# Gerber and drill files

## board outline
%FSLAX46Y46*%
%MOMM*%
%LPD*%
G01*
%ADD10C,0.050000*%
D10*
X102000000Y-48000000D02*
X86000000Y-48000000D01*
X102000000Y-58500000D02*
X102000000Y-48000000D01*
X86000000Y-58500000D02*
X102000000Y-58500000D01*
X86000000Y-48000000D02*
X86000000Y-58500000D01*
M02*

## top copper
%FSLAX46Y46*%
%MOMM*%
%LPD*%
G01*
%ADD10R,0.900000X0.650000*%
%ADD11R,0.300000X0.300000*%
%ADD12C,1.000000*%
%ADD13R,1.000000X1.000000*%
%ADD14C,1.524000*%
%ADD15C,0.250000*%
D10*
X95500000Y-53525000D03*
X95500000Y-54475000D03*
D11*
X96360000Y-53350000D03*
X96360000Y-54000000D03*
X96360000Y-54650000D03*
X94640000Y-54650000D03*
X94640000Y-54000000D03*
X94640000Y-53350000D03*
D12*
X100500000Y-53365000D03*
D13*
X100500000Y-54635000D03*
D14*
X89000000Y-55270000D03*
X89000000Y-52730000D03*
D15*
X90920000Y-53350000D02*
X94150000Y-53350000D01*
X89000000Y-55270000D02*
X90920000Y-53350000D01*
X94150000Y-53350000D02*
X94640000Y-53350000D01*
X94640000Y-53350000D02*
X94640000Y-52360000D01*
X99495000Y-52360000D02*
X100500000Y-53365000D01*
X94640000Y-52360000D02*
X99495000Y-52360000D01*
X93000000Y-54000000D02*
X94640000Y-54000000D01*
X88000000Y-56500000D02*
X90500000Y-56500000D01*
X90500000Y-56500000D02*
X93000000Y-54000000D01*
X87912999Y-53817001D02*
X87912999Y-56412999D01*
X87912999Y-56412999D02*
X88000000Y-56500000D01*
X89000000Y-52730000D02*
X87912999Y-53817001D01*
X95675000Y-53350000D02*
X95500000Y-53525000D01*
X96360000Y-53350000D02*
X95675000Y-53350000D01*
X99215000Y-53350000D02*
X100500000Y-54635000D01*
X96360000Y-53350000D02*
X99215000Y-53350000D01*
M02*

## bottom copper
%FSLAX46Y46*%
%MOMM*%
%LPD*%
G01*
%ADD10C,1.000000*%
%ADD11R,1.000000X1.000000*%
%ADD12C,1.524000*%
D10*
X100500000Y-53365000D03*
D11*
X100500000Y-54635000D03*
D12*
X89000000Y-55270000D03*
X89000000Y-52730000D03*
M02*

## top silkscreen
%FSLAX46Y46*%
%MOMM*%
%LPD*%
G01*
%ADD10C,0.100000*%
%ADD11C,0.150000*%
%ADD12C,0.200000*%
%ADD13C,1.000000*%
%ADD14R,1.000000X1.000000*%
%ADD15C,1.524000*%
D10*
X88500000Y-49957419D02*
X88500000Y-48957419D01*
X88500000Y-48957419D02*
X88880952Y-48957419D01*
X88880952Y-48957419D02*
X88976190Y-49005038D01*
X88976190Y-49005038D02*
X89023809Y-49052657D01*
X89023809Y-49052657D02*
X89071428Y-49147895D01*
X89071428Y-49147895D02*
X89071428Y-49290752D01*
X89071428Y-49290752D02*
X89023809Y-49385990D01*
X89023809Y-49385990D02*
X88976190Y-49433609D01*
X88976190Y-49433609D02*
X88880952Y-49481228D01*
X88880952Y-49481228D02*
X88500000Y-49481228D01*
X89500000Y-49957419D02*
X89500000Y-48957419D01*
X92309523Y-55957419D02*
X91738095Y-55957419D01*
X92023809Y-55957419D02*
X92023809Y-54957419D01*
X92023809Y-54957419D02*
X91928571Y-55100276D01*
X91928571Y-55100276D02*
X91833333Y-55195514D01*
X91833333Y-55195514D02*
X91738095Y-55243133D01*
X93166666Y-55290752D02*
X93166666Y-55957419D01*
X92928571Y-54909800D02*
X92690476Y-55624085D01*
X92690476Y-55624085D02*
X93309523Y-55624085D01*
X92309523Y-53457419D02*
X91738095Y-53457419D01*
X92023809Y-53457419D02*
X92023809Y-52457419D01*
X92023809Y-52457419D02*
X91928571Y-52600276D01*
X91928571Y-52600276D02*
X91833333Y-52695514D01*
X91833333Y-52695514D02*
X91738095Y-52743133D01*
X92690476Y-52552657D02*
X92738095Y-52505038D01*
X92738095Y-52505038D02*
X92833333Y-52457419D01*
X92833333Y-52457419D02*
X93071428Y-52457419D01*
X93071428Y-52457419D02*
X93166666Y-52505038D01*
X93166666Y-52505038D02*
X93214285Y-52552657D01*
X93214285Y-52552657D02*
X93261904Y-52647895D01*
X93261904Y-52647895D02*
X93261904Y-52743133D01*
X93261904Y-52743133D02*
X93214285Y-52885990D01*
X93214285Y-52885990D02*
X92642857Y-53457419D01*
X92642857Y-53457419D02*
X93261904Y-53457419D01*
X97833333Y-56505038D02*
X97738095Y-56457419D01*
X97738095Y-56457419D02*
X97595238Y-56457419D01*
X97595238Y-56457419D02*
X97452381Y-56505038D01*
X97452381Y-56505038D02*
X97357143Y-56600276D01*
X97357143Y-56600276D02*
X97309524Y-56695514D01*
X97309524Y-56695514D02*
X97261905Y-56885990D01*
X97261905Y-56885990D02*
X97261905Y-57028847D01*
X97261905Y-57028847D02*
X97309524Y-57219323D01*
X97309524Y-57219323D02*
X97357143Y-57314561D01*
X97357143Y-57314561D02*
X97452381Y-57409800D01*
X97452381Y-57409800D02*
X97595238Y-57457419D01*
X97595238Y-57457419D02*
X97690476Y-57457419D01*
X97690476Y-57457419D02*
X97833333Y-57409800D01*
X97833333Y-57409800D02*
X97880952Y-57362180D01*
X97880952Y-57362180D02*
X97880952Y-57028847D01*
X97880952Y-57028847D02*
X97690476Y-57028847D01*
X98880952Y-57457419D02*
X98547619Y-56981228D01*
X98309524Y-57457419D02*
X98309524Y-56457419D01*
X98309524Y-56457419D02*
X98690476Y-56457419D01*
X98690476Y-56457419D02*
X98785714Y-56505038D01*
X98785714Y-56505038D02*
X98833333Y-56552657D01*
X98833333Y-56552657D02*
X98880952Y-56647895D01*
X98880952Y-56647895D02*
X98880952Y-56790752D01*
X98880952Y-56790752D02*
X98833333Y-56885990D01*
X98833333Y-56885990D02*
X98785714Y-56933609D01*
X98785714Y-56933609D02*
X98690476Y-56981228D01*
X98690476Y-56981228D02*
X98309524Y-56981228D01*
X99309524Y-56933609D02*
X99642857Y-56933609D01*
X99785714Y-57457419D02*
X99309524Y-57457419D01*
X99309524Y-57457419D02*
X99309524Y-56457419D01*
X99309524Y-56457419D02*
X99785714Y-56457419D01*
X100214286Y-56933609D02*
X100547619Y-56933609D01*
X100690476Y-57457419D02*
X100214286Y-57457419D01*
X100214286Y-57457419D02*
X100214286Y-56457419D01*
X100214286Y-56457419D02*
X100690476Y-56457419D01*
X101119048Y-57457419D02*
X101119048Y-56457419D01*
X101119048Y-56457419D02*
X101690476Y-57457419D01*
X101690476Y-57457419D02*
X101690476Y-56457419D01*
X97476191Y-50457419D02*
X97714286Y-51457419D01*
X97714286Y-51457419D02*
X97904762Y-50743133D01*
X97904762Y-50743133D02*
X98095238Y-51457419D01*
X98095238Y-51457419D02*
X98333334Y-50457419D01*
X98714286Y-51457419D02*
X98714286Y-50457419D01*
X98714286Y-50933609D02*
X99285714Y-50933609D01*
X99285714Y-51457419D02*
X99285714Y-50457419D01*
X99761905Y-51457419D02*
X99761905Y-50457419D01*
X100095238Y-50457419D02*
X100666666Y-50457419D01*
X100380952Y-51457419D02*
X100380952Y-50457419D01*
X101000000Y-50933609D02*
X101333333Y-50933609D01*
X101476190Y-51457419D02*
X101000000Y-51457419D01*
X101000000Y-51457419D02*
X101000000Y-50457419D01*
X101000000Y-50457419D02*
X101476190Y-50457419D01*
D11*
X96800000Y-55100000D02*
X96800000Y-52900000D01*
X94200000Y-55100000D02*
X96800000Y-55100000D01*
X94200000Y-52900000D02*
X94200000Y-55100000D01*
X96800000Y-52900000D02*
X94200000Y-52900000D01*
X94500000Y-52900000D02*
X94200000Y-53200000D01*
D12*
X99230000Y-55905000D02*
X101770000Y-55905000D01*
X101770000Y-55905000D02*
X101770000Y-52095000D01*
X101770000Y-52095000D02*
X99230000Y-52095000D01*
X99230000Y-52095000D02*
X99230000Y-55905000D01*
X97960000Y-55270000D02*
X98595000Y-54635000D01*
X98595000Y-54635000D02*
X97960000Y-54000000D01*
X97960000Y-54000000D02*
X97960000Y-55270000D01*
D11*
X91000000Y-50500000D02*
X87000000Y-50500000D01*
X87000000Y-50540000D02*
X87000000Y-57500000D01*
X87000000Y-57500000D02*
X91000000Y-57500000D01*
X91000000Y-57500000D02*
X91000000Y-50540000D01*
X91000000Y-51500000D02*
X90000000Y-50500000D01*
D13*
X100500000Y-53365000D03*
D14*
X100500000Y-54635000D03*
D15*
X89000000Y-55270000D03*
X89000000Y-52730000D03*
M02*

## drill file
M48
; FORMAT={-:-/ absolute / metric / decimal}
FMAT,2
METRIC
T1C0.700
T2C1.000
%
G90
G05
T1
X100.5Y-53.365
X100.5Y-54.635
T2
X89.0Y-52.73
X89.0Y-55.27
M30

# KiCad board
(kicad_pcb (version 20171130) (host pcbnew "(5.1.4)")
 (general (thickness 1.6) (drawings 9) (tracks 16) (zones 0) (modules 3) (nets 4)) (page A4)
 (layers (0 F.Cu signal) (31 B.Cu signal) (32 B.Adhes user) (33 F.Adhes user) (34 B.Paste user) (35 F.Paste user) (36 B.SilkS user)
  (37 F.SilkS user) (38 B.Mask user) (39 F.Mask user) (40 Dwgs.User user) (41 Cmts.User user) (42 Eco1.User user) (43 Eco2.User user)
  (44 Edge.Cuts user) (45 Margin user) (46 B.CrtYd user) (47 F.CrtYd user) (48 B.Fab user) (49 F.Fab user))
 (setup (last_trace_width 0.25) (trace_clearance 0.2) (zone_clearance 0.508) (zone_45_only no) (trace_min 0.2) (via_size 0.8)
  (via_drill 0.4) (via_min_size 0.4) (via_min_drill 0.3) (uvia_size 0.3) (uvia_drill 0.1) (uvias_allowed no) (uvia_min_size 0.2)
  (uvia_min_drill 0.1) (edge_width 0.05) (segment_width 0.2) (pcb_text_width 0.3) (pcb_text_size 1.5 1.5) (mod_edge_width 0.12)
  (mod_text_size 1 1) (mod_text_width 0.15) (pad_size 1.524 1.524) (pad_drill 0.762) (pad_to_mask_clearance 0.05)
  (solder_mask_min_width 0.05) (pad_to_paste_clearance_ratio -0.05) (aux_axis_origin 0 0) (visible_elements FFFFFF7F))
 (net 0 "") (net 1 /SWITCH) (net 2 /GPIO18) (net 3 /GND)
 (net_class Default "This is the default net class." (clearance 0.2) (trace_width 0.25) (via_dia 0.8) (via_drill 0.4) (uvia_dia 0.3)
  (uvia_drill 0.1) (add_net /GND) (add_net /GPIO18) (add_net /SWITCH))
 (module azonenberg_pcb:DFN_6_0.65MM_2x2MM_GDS (layer F.Cu) (at 95.5 54 270) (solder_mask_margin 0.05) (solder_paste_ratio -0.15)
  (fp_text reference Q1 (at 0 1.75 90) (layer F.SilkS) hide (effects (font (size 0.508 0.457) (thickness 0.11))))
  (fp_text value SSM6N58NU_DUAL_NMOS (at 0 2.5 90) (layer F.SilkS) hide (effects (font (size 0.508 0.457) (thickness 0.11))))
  (fp_line (start 1.1 -1.3) (end -1.1 -1.3) (layer F.SilkS) (width 0.15))
  (fp_line (start 1.1 1.3) (end 1.1 -1.3) (layer F.SilkS) (width 0.15))
  (fp_line (start -1.1 1.3) (end 1.1 1.3) (layer F.SilkS) (width 0.15))
  (fp_line (start -1.1 -1.3) (end -1.1 1.3) (layer F.SilkS) (width 0.15))
  (fp_line (start -1.1 1) (end -0.8 1.3) (layer F.SilkS) (width 0.15))
  (pad D1 smd rect (at -0.475 0 270) (size 0.65 0.9) (layers F.Cu F.Paste F.Mask) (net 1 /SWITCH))
  (pad D2 smd rect (at 0.475 0 270) (size 0.65 0.9) (layers F.Cu F.Paste F.Mask))
  (pad D1 smd rect (at -0.65 -0.86 270) (size 0.3 0.3) (layers F.Cu F.Paste F.Mask) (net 1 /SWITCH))
  (pad G2 smd rect (at 0 -0.86 270) (size 0.3 0.3) (layers F.Cu F.Paste F.Mask))
  (pad S2 smd rect (at 0.65 -0.86 270) (size 0.3 0.3) (layers F.Cu F.Paste F.Mask))
  (pad D2 smd rect (at 0.65 0.86 270) (size 0.3 0.3) (layers F.Cu F.Paste F.Mask))
  (pad G1 smd rect (at 0 0.86 270) (size 0.3 0.3) (layers F.Cu F.Paste F.Mask) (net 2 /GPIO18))
  (pad S1 smd rect (at -0.65 0.86 270) (size 0.3 0.3) (layers F.Cu F.Paste F.Mask) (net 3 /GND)))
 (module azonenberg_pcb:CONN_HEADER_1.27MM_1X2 (layer F.Cu) (at 100.5 54 90)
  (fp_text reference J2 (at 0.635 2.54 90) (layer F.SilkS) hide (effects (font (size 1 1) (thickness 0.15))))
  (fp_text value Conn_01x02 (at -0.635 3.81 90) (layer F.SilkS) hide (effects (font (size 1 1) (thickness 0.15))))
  (fp_line (start -1.905 -1.27) (end -1.905 1.27) (layer F.SilkS) (width 0.2))
  (fp_line (start -1.905 1.27) (end 1.905 1.27) (layer F.SilkS) (width 0.2))
  (fp_line (start 1.905 1.27) (end 1.905 -1.27) (layer F.SilkS) (width 0.2))
  (fp_line (start 1.905 -1.27) (end -1.905 -1.27) (layer F.SilkS) (width 0.2))
  (fp_line (start -1.27 -2.54) (end -0.635 -1.905) (layer F.SilkS) (width 0.2))
  (fp_line (start -0.635 -1.905) (end 0 -2.54) (layer F.SilkS) (width 0.2))
  (fp_line (start 0 -2.54) (end -1.27 -2.54) (layer F.SilkS) (width 0.2))
  (pad 2 thru_hole circle (at 0.635 0 90) (size 1 1) (drill 0.7) (layers *.Cu *.Mask F.SilkS) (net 3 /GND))
  (pad 1 thru_hole rect (at -0.635 0 90) (size 1 1) (drill 0.7) (layers *.Cu *.Mask F.SilkS) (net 1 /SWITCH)))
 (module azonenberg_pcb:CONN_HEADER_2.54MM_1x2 (layer F.Cu) (at 89 54 270)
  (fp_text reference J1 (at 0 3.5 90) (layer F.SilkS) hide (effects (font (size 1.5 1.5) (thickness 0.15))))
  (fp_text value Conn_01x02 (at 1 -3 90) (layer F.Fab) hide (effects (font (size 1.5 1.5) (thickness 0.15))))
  (fp_line (start -3.5 -2) (end -3.5 2) (layer F.SilkS) (width 0.15))
  (fp_line (start -3.46 2) (end 3.5 2) (layer F.SilkS) (width 0.15))
  (fp_line (start 3.5 2) (end 3.5 -2) (layer F.SilkS) (width 0.15))
  (fp_line (start 3.5 -2) (end -3.46 -2) (layer F.SilkS) (width 0.15))
  (fp_line (start -2.5 -2) (end -3.5 -1) (layer F.SilkS) (width 0.15))
  (pad 2 thru_hole circle (at 1.27 0 270) (size 1.524 1.524) (drill 1) (layers *.Cu *.Mask F.SilkS) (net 3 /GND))
  (pad 1 thru_hole circle (at -1.27 0 270) (size 1.524 1.524) (drill 1) (layers *.Cu *.Mask F.SilkS) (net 2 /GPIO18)))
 (gr_line (start 102 48) (end 86 48) (layer Edge.Cuts) (width 0.05))
 (gr_line (start 102 58.5) (end 102 48) (layer Edge.Cuts) (width 0.05))
 (gr_line (start 86 58.5) (end 102 58.5) (layer Edge.Cuts) (width 0.05))
 (gr_line (start 86 48) (end 86 58.5) (layer Edge.Cuts) (width 0.05))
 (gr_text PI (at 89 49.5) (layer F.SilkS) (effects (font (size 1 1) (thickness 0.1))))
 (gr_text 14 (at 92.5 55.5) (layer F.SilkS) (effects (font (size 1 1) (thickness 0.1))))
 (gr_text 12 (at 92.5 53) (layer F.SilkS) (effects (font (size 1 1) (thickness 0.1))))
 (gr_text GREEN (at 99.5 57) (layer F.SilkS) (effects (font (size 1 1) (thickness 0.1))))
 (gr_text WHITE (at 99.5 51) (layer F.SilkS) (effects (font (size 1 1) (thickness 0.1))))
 (segment (start 90.92 53.35) (end 94.15 53.35) (width 0.25) (layer F.Cu) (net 3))
 (segment (start 89 55.27) (end 90.92 53.35) (width 0.25) (layer F.Cu) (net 3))
 (segment (start 94.15 53.35) (end 94.64 53.35) (width 0.25) (layer F.Cu) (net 3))
 (segment (start 94.64 53.35) (end 94.64 52.36) (width 0.25) (layer F.Cu) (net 3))
 (segment (start 99.495 52.36) (end 100.5 53.365) (width 0.25) (layer F.Cu) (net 3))
 (segment (start 94.64 52.36) (end 99.495 52.36) (width 0.25) (layer F.Cu) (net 3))
 (segment (start 93 54) (end 94.64 54) (width 0.25) (layer F.Cu) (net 2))
 (segment (start 88 56.5) (end 90.5 56.5) (width 0.25) (layer F.Cu) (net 2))
 (segment (start 90.5 56.5) (end 93 54) (width 0.25) (layer F.Cu) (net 2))
 (segment (start 87.912999 53.817001) (end 87.912999 56.412999) (width 0.25) (layer F.Cu) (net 2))
 (segment (start 87.912999 56.412999) (end 88 56.5) (width 0.25) (layer F.Cu) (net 2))
 (segment (start 89 52.73) (end 87.912999 53.817001) (width 0.25) (layer F.Cu) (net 2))
 (segment (start 95.675 53.35) (end 95.5 53.525) (width 0.25) (layer F.Cu) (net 1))
 (segment (start 96.36 53.35) (end 95.675 53.35) (width 0.25) (layer F.Cu) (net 1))
 (segment (start 99.215 53.35) (end 100.5 54.635) (width 0.25) (layer F.Cu) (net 1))
 (segment (start 96.36 53.35) (end 99.215 53.35) (width 0.25) (layer F.Cu) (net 1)))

